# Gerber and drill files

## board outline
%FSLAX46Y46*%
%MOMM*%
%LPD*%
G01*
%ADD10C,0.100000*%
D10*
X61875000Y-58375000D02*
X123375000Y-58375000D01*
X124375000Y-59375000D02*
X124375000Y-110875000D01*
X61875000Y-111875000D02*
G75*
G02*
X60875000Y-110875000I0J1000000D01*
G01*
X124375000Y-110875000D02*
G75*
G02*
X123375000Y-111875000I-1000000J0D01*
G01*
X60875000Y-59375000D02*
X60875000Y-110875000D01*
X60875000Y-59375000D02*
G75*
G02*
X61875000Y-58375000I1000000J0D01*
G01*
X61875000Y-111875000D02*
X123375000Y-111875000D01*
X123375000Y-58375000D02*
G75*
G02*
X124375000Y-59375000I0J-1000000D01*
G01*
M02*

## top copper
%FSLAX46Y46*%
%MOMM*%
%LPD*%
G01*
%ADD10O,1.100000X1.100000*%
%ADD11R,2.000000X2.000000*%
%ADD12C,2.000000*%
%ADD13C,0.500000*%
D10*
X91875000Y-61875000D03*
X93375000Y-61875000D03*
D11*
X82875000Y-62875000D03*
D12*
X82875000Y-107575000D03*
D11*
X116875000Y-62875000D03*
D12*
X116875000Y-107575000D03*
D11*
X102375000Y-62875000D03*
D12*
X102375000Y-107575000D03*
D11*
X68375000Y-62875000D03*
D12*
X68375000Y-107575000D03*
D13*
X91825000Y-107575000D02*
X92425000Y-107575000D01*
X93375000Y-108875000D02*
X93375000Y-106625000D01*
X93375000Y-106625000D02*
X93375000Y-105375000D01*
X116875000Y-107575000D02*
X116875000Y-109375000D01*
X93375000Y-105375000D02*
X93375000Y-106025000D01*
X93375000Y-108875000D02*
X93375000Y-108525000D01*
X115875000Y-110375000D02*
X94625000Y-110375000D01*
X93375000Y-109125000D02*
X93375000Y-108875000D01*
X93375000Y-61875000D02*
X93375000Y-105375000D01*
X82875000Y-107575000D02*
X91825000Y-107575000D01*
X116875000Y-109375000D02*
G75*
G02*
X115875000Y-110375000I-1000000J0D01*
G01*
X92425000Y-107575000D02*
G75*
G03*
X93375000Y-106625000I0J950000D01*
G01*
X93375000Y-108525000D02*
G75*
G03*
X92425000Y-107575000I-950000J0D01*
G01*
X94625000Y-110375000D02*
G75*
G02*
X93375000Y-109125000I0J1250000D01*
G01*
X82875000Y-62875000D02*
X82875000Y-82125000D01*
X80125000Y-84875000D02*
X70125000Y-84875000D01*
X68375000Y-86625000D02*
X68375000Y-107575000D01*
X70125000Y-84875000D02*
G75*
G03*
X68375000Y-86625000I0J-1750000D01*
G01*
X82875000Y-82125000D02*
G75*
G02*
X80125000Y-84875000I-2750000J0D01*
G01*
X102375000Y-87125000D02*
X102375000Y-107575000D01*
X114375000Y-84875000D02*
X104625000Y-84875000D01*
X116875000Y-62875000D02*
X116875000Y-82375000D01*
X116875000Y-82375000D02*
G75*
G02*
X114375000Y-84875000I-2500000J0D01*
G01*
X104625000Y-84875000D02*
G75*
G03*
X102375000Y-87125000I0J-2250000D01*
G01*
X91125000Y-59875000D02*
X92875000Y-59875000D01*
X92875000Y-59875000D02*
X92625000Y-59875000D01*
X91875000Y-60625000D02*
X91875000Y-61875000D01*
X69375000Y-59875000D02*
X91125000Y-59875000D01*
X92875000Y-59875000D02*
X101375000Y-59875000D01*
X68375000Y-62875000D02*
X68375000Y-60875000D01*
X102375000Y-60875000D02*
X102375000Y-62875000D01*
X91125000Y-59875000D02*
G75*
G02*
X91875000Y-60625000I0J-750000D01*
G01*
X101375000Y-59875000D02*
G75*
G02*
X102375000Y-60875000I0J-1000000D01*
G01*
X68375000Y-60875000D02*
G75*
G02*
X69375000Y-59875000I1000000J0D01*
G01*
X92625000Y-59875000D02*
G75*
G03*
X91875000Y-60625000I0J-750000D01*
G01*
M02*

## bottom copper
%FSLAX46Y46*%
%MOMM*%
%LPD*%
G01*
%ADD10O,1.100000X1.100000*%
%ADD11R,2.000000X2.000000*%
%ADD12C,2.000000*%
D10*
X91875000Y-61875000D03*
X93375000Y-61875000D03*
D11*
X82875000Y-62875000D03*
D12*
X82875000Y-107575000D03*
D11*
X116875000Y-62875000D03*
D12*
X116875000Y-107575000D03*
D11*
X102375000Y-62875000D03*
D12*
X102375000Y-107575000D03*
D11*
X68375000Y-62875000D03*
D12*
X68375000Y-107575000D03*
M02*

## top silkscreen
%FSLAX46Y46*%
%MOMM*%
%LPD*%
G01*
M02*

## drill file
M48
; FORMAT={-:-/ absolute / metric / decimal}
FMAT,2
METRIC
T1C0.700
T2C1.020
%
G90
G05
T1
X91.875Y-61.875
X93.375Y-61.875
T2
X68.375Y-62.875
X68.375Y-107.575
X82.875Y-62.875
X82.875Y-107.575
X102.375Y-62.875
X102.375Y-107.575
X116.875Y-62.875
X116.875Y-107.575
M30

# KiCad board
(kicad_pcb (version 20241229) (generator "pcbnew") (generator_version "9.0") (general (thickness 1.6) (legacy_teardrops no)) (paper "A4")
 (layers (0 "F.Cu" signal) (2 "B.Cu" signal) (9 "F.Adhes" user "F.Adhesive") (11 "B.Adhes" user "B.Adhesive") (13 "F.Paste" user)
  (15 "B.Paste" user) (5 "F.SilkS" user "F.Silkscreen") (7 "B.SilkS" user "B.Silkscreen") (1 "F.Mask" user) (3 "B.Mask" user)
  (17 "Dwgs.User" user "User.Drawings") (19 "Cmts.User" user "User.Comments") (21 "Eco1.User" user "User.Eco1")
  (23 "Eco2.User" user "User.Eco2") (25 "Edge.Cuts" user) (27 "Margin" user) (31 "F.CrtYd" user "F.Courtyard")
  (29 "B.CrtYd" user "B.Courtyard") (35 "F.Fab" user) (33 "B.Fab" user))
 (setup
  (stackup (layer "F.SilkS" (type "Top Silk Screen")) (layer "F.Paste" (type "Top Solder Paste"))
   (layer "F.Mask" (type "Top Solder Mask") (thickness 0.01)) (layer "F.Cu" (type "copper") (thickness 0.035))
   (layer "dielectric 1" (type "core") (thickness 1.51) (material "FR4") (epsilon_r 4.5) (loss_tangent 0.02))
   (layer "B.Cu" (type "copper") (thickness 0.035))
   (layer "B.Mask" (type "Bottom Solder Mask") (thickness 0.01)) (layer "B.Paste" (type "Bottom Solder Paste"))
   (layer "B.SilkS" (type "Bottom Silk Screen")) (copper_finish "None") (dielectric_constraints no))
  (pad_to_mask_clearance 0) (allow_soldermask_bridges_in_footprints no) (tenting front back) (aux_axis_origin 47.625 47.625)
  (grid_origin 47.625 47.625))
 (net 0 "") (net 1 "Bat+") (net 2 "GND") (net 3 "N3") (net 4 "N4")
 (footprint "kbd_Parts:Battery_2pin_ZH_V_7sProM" (layer "F.Cu") (at 92.625 61.875)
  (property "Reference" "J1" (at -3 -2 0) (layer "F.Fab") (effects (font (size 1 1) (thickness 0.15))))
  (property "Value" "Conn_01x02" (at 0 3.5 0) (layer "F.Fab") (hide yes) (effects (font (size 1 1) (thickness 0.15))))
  (pad "1" thru_hole oval (at -0.75 0) (size 1.1 1.1) (drill oval 0.7) (layers "*.Cu" "*.Mask") (remove_unused_layers no) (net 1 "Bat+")
   (clearance 0.15))
  (pad "2" thru_hole oval (at 0.75 0) (size 1.1 1.1) (drill oval 0.7) (layers "*.Cu" "*.Mask") (remove_unused_layers no) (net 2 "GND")
   (clearance 0.15)))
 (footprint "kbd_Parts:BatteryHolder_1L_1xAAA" (layer "B.Cu") (at 82.875 62.875 -90)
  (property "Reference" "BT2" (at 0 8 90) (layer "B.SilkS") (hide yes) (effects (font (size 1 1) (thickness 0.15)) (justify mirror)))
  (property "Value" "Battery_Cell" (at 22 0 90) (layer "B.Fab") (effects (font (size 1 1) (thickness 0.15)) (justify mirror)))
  (pad "1" thru_hole rect (at 0 0 270) (size 2 2) (drill 1.02) (layers "*.Cu" "*.Mask") (remove_unused_layers no) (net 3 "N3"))
  (pad "2" thru_hole circle (at 44.7 0 270) (size 2 2) (drill 1.02) (layers "*.Cu" "*.Mask") (remove_unused_layers no) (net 2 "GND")))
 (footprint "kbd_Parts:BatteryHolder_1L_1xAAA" (layer "B.Cu") (at 116.875 62.875 -90)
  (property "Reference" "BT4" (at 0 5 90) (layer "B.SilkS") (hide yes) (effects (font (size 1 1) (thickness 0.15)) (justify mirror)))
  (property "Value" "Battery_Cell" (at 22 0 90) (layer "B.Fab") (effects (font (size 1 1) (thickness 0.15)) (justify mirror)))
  (pad "1" thru_hole rect (at 0 0 270) (size 2 2) (drill 1.02) (layers "*.Cu" "*.Mask") (remove_unused_layers no) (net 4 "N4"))
  (pad "2" thru_hole circle (at 44.7 0 270) (size 2 2) (drill 1.02) (layers "*.Cu" "*.Mask") (remove_unused_layers no) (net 2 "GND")))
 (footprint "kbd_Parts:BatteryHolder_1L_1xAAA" (layer "B.Cu") (at 102.375 62.875 -90)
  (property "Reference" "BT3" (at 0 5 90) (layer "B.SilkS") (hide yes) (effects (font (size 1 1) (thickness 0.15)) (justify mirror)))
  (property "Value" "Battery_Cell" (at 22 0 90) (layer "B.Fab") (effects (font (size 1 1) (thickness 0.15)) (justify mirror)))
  (pad "1" thru_hole rect (at 0 0 270) (size 2 2) (drill 1.02) (layers "*.Cu" "*.Mask") (remove_unused_layers no) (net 1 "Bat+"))
  (pad "2" thru_hole circle (at 44.7 0 270) (size 2 2) (drill 1.02) (layers "*.Cu" "*.Mask") (remove_unused_layers no) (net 4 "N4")))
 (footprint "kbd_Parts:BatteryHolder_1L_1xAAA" (layer "B.Cu") (at 68.375 62.875 -90)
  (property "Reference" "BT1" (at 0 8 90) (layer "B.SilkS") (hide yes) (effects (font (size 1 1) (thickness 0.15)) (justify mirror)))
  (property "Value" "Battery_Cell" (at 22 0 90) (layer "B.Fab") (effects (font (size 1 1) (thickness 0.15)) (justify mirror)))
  (pad "1" thru_hole rect (at 0 0 270) (size 2 2) (drill 1.02) (layers "*.Cu" "*.Mask") (remove_unused_layers no) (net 1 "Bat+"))
  (pad "2" thru_hole circle (at 44.7 0 270) (size 2 2) (drill 1.02) (layers "*.Cu" "*.Mask") (remove_unused_layers no) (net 3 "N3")))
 (gr_line (start 61.875 58.375) (end 123.375 58.375) (stroke (width 0.1) (type solid)) (layer "Edge.Cuts"))
 (gr_line (start 124.375 59.375) (end 124.375 110.875) (stroke (width 0.1) (type solid)) (layer "Edge.Cuts"))
 (gr_arc (start 61.875 111.875) (mid 61.167893 111.582107) (end 60.875 110.875) (stroke (width 0.1) (type solid)) (layer "Edge.Cuts"))
 (gr_arc (start 124.375 110.875) (mid 124.082107 111.582107) (end 123.375 111.875) (stroke (width 0.1) (type solid)) (layer "Edge.Cuts"))
 (gr_line (start 60.875 59.375) (end 60.875 110.875) (stroke (width 0.1) (type solid)) (layer "Edge.Cuts"))
 (gr_arc (start 60.875 59.375) (mid 61.167893 58.667893) (end 61.875 58.375) (stroke (width 0.1) (type solid)) (layer "Edge.Cuts"))
 (gr_line (start 61.875 111.875) (end 123.375 111.875) (stroke (width 0.1) (type solid)) (layer "Edge.Cuts"))
 (gr_arc (start 123.375 58.375) (mid 124.082107 58.667893) (end 124.375 59.375) (stroke (width 0.1) (type solid)) (layer "Edge.Cuts"))
 (segment (start 91.825 107.575) (end 92.425 107.575) (width 0.5) (layer "F.Cu") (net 2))
 (segment (start 93.375 108.875) (end 93.375 106.625) (width 0.5) (layer "F.Cu") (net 2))
 (segment (start 93.375 106.625) (end 93.375 105.375) (width 0.5) (layer "F.Cu") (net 2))
 (segment (start 116.875 107.575) (end 116.875 109.375) (width 0.5) (layer "F.Cu") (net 2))
 (segment (start 93.375 105.375) (end 93.375 106.025) (width 0.5) (layer "F.Cu") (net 2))
 (segment (start 93.375 108.875) (end 93.375 108.525) (width 0.5) (layer "F.Cu") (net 2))
 (segment (start 115.875 110.375) (end 94.625 110.375) (width 0.5) (layer "F.Cu") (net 2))
 (segment (start 93.375 109.125) (end 93.375 108.875) (width 0.5) (layer "F.Cu") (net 2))
 (segment (start 93.375 61.875) (end 93.375 105.375) (width 0.5) (layer "F.Cu") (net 2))
 (segment (start 82.875 107.575) (end 91.825 107.575) (width 0.5) (layer "F.Cu") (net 2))
 (arc (start 116.875 109.375) (mid 116.582107 110.082107) (end 115.875 110.375) (width 0.5) (layer "F.Cu") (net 2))
 (arc (start 92.425 107.575) (mid 93.096751 107.296751) (end 93.375 106.625) (width 0.5) (layer "F.Cu") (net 2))
 (arc (start 93.375 108.525) (mid 93.096751 107.853249) (end 92.425 107.575) (width 0.5) (layer "F.Cu") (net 2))
 (arc (start 94.625 110.375) (mid 93.741117 110.008883) (end 93.375 109.125) (width 0.5) (layer "F.Cu") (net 2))
 (segment (start 82.875 62.875) (end 82.875 82.125) (width 0.5) (layer "F.Cu") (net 3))
 (segment (start 80.125 84.875) (end 70.125 84.875) (width 0.5) (layer "F.Cu") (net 3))
 (segment (start 68.375 86.625) (end 68.375 107.575) (width 0.5) (layer "F.Cu") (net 3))
 (arc (start 70.125 84.875) (mid 68.887563 85.387563) (end 68.375 86.625) (width 0.5) (layer "F.Cu") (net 3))
 (arc (start 82.875 82.125) (mid 82.069544 84.069544) (end 80.125 84.875) (width 0.5) (layer "F.Cu") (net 3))
 (segment (start 102.375 87.125) (end 102.375 107.575) (width 0.5) (layer "F.Cu") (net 4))
 (segment (start 114.375 84.875) (end 104.625 84.875) (width 0.5) (layer "F.Cu") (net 4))
 (segment (start 116.875 62.875) (end 116.875 82.375) (width 0.5) (layer "F.Cu") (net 4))
 (arc (start 116.875 82.375) (mid 116.142767 84.142767) (end 114.375 84.875) (width 0.5) (layer "F.Cu") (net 4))
 (arc (start 104.625 84.875) (mid 103.03401 85.53401) (end 102.375 87.125) (width 0.5) (layer "F.Cu") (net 4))
 (segment (start 91.125 59.875) (end 92.875 59.875) (width 0.5) (layer "F.Cu") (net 1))
 (segment (start 92.875 59.875) (end 92.625 59.875) (width 0.5) (layer "F.Cu") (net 1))
 (segment (start 91.875 60.625) (end 91.875 61.875) (width 0.5) (layer "F.Cu") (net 1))
 (segment (start 69.375 59.875) (end 91.125 59.875) (width 0.5) (layer "F.Cu") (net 1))
 (segment (start 92.875 59.875) (end 101.375 59.875) (width 0.5) (layer "F.Cu") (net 1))
 (segment (start 68.375 62.875) (end 68.375 60.875) (width 0.5) (layer "F.Cu") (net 1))
 (segment (start 102.375 60.875) (end 102.375 62.875) (width 0.5) (layer "F.Cu") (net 1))
 (arc (start 91.125 59.875) (mid 91.65533 60.09467) (end 91.875 60.625) (width 0.5) (layer "F.Cu") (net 1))
 (arc (start 101.375 59.875) (mid 102.082107 60.167893) (end 102.375 60.875) (width 0.5) (layer "F.Cu") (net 1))
 (arc (start 68.375 60.875) (mid 68.667893 60.167893) (end 69.375 59.875) (width 0.5) (layer "F.Cu") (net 1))
 (arc (start 92.625 59.875) (mid 92.09467 60.09467) (end 91.875 60.625) (width 0.5) (layer "F.Cu") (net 1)))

